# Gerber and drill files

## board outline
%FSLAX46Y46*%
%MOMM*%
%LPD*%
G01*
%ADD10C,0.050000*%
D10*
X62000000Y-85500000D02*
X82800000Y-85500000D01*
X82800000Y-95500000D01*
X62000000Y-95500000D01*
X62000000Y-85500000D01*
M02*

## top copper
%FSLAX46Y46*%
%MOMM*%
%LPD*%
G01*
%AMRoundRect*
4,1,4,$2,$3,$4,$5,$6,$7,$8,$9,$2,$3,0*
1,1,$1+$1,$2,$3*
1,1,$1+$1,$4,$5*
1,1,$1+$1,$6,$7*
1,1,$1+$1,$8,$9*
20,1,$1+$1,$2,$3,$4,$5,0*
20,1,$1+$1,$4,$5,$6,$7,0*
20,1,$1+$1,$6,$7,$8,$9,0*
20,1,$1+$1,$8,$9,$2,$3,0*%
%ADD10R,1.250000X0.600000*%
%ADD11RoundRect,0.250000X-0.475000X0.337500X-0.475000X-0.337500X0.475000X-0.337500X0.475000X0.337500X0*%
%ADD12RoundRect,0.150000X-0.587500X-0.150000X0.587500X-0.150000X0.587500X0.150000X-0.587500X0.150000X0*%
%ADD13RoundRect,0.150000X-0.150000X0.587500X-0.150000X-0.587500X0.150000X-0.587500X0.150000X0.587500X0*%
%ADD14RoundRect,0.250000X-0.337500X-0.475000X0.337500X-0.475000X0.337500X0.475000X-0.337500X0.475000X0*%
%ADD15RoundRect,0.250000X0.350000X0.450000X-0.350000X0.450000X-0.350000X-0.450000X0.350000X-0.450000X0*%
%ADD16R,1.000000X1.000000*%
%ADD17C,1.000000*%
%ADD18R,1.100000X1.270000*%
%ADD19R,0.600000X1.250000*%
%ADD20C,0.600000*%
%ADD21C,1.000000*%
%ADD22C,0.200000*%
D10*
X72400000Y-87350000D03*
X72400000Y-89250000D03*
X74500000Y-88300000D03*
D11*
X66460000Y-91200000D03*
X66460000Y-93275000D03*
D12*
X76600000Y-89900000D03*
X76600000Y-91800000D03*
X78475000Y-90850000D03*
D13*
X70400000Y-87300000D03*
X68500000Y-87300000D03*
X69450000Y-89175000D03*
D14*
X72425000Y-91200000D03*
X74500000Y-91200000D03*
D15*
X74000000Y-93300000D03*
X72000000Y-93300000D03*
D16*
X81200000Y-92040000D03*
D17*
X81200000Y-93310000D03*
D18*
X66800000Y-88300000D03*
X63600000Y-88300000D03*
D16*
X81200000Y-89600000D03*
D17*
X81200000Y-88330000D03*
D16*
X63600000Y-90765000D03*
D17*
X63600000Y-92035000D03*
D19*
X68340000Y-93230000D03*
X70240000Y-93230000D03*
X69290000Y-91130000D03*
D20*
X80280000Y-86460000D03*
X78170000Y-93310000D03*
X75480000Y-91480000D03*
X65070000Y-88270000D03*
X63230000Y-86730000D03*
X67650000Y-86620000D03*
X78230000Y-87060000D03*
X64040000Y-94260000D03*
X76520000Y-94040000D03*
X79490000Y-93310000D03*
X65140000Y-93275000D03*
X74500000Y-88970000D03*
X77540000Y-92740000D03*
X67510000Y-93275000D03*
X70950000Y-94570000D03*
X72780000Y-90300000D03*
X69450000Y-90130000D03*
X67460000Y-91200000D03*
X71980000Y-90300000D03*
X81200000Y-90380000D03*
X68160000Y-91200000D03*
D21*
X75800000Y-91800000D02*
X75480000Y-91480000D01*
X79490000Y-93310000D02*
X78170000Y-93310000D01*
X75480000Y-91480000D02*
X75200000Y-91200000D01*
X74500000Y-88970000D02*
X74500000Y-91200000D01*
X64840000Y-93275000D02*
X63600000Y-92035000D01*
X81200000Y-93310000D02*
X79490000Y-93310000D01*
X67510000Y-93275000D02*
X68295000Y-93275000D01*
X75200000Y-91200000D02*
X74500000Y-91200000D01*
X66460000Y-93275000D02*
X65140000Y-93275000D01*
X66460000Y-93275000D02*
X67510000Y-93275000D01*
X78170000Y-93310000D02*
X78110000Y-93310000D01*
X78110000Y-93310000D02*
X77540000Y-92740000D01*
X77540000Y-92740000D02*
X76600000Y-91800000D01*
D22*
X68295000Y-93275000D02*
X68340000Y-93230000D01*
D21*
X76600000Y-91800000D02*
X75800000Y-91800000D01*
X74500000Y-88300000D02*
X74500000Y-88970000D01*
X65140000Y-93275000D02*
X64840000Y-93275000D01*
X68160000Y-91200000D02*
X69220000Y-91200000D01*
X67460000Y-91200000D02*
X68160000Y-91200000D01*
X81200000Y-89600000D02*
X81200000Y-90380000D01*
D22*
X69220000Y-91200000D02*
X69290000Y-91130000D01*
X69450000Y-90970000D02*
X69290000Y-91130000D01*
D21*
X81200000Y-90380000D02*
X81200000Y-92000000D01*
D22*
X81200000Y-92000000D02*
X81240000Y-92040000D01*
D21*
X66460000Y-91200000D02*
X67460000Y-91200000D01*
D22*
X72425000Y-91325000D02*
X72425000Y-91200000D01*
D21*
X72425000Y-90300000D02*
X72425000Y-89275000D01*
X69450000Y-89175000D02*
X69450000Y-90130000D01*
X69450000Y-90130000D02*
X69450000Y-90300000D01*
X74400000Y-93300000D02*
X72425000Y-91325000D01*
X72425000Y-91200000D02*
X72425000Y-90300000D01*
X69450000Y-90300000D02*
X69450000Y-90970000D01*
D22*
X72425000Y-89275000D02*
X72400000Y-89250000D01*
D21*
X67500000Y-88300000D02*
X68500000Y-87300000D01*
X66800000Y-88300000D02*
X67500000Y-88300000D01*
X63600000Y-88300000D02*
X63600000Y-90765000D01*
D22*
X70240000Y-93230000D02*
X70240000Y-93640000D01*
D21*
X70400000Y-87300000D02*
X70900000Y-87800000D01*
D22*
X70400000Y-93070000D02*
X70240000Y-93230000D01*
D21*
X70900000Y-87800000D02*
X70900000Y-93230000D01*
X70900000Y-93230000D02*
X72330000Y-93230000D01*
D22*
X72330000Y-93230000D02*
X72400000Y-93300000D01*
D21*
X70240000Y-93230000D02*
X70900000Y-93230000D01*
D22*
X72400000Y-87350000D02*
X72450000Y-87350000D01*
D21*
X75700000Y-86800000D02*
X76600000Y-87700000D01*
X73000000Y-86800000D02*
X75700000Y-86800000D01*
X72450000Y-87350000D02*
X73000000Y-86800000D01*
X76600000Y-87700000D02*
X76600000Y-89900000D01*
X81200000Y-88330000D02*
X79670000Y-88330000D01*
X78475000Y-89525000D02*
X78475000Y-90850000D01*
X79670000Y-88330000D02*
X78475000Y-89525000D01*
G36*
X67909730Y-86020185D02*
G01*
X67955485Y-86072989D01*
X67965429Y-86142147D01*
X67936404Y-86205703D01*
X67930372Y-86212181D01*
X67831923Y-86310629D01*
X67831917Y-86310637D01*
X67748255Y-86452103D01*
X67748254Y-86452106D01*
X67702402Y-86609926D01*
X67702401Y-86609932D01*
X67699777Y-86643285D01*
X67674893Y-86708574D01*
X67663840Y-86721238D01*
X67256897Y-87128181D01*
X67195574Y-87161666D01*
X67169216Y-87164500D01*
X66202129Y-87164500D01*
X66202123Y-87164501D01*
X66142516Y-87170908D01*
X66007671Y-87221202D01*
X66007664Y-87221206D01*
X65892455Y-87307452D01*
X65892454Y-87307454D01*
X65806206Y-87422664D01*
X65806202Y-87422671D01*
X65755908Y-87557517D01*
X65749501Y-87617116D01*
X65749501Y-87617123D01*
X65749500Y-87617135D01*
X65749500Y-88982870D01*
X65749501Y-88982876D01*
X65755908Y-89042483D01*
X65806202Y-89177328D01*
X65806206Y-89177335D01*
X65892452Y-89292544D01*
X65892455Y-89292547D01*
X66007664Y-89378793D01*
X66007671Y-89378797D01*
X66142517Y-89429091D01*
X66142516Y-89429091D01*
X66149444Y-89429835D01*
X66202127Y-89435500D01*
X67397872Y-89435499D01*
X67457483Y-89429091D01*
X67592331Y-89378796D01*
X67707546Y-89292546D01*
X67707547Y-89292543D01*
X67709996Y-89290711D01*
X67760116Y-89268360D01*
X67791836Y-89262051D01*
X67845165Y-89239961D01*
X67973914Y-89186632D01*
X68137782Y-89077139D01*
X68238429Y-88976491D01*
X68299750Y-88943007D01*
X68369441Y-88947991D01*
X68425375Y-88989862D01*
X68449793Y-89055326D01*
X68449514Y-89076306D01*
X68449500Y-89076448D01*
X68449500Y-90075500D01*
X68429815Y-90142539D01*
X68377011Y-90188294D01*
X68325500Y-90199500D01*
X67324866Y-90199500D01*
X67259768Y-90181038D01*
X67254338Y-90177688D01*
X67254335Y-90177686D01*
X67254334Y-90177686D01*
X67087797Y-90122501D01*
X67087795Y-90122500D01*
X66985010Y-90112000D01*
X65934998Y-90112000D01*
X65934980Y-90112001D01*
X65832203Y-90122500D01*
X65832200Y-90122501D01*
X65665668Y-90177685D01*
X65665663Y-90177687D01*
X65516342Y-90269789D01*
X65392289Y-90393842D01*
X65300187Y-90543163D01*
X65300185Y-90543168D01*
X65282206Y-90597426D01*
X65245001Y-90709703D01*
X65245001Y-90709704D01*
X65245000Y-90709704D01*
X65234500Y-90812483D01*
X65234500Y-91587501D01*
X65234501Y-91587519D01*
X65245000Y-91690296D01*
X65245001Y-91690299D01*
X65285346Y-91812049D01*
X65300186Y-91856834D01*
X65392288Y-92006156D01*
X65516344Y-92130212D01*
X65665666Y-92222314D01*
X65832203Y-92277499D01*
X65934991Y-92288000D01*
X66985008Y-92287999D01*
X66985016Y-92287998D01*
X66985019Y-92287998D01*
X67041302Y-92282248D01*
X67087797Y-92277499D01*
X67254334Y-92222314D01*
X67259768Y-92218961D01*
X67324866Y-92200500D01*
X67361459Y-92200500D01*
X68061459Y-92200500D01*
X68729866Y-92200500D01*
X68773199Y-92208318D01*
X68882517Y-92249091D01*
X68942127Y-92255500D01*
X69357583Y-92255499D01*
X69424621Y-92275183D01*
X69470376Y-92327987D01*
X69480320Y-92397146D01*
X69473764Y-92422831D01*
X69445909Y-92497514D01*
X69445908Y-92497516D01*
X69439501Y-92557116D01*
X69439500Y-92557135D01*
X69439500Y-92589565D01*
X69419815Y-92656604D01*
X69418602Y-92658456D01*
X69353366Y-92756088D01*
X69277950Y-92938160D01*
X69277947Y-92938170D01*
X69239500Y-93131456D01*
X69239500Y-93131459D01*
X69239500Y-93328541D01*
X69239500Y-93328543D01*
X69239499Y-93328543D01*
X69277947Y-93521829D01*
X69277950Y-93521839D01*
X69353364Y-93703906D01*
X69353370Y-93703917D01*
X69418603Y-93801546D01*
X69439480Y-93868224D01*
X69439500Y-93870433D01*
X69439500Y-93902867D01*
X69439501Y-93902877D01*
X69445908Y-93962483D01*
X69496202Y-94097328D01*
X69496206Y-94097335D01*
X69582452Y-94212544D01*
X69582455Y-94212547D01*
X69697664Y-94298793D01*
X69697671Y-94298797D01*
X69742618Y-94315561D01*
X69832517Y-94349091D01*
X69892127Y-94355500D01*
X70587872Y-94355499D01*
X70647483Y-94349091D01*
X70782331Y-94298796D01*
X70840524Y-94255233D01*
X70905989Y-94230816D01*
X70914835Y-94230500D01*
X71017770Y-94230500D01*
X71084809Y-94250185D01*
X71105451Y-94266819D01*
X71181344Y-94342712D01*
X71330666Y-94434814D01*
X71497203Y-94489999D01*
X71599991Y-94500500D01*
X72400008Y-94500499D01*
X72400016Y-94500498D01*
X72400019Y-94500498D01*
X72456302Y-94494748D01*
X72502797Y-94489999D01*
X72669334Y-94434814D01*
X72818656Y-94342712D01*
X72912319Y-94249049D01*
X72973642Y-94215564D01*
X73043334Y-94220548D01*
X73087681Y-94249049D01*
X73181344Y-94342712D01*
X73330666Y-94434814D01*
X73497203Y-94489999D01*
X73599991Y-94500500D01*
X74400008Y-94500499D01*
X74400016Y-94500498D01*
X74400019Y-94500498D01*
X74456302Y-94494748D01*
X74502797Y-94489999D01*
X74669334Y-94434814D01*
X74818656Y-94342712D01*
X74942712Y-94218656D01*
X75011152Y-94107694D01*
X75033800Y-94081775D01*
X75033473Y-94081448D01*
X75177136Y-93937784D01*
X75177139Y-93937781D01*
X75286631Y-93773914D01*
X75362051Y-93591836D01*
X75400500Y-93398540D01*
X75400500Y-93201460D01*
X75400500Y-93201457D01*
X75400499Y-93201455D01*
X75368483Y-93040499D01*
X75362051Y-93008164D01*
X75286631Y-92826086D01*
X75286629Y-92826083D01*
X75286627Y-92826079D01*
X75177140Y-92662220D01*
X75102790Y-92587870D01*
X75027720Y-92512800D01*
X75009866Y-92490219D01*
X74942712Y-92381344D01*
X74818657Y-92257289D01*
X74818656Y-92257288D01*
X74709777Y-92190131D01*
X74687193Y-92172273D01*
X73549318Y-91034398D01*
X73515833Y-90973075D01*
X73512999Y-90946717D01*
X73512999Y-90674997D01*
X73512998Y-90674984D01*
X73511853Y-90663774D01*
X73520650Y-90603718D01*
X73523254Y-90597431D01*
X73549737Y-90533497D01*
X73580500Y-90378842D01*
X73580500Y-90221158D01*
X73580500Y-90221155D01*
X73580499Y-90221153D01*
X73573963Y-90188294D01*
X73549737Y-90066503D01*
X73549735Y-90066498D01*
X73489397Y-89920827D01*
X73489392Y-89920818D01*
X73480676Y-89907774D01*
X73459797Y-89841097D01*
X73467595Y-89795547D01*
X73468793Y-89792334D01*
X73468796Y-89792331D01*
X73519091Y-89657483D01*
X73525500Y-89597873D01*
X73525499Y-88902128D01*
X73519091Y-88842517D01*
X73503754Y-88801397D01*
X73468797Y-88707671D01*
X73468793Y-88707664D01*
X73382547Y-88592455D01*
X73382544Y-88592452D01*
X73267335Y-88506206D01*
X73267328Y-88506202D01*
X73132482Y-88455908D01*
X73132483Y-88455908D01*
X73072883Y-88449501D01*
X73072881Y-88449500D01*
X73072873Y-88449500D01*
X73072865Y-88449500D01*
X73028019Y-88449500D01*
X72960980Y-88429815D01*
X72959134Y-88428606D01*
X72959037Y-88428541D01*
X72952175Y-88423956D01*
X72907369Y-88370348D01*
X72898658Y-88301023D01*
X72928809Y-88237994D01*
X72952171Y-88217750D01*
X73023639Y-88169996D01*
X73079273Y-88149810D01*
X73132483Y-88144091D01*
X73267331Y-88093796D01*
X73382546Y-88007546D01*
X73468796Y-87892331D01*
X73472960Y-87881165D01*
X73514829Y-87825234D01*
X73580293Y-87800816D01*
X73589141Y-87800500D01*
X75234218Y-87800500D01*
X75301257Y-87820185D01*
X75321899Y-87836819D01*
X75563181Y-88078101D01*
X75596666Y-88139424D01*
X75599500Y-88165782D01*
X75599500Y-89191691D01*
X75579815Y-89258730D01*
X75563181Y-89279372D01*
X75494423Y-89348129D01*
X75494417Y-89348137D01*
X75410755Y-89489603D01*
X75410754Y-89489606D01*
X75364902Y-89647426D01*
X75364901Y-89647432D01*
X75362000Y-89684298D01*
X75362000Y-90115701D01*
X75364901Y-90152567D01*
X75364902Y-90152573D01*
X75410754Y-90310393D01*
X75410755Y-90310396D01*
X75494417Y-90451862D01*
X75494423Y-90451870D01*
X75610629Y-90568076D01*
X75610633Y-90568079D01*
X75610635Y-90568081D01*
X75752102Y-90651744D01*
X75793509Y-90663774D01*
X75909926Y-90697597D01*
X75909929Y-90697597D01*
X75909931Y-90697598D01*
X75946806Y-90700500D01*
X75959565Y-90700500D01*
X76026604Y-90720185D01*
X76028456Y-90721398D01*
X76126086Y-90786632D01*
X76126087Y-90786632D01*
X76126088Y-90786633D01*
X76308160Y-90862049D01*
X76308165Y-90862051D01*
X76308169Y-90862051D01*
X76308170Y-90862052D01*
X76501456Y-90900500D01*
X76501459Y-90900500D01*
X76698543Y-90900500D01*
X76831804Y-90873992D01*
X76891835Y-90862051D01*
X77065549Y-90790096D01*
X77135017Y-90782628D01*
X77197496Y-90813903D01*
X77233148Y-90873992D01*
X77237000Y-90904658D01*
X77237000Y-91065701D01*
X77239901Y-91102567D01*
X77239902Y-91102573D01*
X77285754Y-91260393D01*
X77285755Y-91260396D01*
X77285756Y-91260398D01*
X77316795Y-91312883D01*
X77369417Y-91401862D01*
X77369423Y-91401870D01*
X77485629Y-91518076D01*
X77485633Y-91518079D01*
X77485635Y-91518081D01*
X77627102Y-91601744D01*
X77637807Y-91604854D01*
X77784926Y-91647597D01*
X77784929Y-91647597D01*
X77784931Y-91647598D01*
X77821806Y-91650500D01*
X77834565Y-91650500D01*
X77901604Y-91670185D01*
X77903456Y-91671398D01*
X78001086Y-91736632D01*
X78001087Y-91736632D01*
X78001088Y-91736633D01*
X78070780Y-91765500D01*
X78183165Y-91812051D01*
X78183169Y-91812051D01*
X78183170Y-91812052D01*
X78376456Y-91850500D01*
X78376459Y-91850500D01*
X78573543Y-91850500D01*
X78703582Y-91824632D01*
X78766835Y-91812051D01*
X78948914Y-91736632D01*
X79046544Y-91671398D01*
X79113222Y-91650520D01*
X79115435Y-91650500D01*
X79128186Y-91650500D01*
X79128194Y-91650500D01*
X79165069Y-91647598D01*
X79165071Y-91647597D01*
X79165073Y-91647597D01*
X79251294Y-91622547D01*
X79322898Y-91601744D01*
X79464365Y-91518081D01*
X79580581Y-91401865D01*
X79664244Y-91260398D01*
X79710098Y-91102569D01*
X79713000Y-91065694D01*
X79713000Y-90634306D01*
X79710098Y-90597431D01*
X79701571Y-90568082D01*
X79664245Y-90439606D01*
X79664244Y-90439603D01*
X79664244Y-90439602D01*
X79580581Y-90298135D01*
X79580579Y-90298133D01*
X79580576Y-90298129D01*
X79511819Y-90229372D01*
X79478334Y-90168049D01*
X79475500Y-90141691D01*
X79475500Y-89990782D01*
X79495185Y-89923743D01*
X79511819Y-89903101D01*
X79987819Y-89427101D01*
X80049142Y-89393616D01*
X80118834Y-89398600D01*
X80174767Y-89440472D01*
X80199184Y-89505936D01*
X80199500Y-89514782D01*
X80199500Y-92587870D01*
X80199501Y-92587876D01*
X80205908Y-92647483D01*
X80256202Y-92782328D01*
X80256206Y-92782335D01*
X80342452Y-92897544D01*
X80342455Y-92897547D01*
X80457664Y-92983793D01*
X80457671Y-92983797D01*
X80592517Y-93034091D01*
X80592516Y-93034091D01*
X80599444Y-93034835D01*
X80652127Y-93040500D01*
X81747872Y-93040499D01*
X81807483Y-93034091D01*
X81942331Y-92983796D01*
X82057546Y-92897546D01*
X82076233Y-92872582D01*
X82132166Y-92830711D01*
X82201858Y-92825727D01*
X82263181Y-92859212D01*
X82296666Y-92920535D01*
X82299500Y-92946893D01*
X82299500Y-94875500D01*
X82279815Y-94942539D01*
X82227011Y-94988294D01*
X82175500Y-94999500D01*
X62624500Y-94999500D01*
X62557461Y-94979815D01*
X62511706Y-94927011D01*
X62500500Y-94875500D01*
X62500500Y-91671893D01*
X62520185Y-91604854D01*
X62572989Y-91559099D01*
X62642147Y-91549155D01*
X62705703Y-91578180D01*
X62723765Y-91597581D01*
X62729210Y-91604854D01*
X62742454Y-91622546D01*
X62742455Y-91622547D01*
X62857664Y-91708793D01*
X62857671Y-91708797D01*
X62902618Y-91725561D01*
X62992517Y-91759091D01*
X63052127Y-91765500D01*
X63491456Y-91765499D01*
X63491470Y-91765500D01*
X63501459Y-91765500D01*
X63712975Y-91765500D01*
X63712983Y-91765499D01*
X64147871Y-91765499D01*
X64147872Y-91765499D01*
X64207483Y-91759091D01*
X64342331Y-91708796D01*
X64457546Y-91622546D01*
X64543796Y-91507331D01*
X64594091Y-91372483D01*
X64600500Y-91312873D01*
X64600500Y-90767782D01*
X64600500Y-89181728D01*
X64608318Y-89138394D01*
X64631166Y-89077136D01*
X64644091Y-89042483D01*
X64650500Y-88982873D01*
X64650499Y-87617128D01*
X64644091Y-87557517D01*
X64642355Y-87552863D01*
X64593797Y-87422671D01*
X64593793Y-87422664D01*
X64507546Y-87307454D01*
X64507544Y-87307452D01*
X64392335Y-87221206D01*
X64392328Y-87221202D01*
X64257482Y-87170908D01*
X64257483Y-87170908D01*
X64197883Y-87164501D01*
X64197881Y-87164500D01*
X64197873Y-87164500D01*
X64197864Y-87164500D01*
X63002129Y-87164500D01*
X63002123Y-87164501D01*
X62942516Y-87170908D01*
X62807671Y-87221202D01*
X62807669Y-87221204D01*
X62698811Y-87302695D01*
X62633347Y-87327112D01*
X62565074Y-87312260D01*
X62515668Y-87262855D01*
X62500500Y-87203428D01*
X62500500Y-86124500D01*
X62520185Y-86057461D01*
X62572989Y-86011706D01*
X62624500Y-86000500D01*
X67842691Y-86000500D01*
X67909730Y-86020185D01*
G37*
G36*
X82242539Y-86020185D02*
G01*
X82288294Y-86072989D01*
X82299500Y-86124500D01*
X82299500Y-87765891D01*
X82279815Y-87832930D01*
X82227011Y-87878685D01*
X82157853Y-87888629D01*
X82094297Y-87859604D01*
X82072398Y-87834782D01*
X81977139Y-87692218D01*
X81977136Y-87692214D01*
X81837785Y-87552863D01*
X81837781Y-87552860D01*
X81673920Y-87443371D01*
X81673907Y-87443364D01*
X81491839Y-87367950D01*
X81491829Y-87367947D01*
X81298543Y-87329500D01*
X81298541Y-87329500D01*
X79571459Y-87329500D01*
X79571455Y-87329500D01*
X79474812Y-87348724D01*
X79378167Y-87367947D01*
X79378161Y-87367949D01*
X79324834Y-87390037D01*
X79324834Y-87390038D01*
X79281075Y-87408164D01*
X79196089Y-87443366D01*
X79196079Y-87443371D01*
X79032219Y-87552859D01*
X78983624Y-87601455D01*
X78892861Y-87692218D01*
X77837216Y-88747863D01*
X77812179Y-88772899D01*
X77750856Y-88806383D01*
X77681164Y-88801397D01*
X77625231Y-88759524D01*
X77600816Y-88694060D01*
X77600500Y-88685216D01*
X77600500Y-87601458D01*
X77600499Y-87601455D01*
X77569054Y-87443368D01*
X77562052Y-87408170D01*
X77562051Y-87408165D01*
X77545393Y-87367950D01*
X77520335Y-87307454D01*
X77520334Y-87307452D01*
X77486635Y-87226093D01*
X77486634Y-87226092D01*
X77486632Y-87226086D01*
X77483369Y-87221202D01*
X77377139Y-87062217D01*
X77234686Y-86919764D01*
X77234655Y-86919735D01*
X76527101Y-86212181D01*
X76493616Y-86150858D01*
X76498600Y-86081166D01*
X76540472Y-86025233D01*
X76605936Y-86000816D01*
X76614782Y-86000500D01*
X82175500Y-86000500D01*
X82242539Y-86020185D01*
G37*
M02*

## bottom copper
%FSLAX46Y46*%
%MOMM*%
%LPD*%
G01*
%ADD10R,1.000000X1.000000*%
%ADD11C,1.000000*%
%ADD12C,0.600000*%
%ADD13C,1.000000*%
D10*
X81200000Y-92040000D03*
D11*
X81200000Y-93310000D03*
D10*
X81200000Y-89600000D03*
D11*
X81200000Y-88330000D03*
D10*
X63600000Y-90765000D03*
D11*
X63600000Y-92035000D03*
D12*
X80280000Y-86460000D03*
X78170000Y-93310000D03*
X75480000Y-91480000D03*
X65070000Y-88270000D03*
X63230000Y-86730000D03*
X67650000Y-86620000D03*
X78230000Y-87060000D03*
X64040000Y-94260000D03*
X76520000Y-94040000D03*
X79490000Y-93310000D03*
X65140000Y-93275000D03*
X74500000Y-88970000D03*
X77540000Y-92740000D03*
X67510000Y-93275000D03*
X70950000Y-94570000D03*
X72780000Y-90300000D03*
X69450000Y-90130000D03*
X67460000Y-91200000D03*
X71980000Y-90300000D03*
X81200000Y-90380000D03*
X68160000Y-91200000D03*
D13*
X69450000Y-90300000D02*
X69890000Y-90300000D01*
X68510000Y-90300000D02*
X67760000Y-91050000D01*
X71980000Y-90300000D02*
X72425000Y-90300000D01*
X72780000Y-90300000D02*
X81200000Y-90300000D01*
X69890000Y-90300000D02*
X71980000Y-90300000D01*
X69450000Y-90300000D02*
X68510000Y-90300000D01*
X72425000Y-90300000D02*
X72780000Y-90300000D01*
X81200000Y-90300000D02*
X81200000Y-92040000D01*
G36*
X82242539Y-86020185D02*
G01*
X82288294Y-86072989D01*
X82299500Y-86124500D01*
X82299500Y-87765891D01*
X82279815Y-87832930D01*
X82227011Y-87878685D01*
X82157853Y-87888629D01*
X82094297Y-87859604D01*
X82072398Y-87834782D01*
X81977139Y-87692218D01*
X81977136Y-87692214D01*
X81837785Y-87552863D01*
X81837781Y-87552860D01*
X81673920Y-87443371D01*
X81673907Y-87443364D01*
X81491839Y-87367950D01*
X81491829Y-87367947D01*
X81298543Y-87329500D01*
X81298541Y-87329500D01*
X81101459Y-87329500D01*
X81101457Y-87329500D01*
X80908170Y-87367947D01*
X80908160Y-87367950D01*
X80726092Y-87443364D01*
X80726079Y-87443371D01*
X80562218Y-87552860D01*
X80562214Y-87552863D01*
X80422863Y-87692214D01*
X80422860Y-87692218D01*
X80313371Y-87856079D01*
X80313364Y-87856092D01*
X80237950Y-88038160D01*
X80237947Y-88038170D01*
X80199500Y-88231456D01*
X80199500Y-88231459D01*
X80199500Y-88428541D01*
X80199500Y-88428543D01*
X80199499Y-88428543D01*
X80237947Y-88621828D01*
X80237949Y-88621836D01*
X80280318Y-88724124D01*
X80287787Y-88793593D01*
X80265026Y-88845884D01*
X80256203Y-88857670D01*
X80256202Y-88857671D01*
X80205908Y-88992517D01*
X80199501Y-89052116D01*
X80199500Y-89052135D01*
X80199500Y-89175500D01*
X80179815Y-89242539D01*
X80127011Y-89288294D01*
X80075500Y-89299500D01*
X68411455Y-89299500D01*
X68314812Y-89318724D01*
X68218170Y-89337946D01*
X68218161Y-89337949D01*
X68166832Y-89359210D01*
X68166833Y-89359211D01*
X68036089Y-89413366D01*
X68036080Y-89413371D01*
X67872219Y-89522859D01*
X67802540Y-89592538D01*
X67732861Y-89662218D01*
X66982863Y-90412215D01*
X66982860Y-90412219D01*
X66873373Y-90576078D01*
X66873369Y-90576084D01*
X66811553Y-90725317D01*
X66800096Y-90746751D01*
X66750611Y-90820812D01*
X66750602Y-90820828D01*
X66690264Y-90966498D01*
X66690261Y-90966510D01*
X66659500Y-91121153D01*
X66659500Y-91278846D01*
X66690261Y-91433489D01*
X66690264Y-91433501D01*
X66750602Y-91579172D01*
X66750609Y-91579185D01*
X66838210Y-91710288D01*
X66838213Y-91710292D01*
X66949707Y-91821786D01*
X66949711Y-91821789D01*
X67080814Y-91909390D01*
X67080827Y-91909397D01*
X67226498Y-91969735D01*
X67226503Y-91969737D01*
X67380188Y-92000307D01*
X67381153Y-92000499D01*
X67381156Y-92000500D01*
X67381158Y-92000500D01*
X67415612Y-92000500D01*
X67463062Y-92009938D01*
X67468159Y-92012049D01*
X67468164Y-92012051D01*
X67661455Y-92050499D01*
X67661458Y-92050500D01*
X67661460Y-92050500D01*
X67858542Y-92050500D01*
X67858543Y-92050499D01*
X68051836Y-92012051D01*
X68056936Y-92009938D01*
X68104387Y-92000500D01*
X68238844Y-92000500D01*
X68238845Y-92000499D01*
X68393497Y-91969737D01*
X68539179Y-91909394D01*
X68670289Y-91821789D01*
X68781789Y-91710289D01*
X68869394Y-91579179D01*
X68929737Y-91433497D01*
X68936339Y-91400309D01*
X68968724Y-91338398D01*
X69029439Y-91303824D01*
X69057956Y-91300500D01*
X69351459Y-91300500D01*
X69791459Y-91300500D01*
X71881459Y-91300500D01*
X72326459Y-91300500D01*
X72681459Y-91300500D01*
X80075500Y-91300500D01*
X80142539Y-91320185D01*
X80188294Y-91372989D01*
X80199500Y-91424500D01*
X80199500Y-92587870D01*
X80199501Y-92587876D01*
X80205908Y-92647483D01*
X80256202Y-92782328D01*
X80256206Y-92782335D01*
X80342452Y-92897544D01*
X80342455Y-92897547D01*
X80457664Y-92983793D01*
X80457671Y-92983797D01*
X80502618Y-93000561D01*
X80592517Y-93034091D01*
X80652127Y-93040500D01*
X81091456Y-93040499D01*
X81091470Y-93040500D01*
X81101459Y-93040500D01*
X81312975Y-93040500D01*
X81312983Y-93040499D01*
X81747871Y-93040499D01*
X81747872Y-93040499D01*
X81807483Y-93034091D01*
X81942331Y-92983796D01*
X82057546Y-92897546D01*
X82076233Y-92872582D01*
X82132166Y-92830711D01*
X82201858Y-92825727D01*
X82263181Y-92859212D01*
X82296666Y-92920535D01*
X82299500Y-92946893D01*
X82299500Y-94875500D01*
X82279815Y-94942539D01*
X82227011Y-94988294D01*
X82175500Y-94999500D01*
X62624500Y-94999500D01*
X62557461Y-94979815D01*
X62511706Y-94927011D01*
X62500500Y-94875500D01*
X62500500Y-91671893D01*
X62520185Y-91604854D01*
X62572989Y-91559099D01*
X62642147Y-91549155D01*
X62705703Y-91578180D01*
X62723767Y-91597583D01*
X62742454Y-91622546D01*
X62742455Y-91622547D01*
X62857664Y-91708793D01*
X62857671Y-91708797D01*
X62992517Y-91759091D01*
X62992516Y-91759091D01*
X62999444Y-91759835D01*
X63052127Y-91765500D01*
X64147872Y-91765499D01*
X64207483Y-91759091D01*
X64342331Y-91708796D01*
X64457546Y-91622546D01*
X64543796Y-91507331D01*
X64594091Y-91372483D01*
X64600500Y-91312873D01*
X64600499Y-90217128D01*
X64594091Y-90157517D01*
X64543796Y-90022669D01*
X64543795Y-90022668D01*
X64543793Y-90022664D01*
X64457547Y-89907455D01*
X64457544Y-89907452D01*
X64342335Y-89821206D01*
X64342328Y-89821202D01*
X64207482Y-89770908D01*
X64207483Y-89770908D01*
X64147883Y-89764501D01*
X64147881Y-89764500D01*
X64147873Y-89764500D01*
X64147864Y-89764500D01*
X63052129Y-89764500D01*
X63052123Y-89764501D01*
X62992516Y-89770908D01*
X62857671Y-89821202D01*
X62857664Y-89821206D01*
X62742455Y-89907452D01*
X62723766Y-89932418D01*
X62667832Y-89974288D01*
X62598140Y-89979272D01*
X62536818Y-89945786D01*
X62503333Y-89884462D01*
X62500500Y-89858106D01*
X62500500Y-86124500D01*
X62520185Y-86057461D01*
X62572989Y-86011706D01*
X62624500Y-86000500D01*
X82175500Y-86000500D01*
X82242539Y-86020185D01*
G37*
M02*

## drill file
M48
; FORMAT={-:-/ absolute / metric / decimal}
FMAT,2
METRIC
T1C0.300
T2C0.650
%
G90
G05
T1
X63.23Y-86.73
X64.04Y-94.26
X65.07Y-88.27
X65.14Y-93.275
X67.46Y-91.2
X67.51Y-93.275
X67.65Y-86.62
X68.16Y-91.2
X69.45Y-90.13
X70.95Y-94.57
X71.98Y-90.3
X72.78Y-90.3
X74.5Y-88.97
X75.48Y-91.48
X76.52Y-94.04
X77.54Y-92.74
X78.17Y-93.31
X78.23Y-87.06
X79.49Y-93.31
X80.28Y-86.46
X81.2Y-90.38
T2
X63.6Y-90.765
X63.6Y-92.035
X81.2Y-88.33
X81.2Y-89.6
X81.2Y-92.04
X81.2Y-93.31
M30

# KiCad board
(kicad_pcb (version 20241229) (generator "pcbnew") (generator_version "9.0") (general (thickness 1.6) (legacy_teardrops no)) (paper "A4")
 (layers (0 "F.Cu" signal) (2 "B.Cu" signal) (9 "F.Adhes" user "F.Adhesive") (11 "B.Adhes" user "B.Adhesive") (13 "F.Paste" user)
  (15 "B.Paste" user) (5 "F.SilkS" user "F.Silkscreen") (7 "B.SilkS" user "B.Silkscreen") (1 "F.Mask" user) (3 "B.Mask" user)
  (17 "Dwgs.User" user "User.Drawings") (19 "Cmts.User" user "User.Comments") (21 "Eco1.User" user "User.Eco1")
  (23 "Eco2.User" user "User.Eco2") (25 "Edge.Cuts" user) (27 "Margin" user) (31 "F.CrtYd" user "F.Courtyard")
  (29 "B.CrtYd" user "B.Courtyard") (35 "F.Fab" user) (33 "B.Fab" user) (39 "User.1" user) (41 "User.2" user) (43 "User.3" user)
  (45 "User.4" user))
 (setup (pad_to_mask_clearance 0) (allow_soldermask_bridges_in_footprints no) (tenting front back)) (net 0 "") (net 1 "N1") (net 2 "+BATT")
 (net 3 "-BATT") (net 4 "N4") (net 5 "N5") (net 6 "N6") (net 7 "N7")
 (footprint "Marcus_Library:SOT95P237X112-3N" (layer "F.Cu") (at 73.45 88.3)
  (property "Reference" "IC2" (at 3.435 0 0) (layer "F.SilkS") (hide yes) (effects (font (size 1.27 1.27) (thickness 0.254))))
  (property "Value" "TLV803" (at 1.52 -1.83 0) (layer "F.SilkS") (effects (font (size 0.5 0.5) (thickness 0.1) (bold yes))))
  (pad "1" smd rect (at -1.05 -0.95 90) (size 0.6 1.25) (layers "F.Cu" "F.Mask" "F.Paste") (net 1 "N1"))
  (pad "2" smd rect (at -1.05 0.95 90) (size 0.6 1.25) (layers "F.Cu" "F.Mask" "F.Paste") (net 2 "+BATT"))
  (pad "3" smd rect (at 1.05 0 90) (size 0.6 1.25) (layers "F.Cu" "F.Mask" "F.Paste") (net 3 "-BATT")))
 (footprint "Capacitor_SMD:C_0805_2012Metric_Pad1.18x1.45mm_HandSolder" (layer "F.Cu") (at 66.46 92.2375 -90)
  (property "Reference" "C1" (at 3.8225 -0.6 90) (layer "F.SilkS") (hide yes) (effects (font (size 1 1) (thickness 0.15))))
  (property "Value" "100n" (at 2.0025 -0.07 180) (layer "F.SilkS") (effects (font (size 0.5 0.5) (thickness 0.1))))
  (pad "1" smd roundrect (at -1.0375 0 270) (size 1.175 1.45) (layers "F.Cu" "F.Mask" "F.Paste") (roundrect_rratio 0.212766) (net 2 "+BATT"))
  (pad "2" smd roundrect (at 1.0375 0 270) (size 1.175 1.45) (layers "F.Cu" "F.Mask" "F.Paste") (roundrect_rratio 0.212766) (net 3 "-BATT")))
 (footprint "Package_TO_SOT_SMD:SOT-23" (layer "F.Cu") (at 77.5375 90.85)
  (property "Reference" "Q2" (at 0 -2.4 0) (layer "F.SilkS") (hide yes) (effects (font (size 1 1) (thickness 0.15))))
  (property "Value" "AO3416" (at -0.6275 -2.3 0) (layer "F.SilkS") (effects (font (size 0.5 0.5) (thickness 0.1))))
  (pad "1" smd roundrect (at -0.9375 -0.95) (size 1.475 0.6) (layers "F.Cu" "F.Mask" "F.Paste") (roundrect_rratio 0.25) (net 1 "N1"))
  (pad "2" smd roundrect (at -0.9375 0.95) (size 1.475 0.6) (layers "F.Cu" "F.Mask" "F.Paste") (roundrect_rratio 0.25) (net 3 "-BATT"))
  (pad "3" smd roundrect (at 0.9375 0) (size 1.475 0.6) (layers "F.Cu" "F.Mask" "F.Paste") (roundrect_rratio 0.25) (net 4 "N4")))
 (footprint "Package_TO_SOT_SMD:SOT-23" (layer "F.Cu") (at 69.45 88.2375 -90)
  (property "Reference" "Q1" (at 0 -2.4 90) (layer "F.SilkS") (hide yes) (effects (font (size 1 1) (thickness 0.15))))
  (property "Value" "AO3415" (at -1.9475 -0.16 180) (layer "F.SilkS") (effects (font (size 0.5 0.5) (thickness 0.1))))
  (pad "1" smd roundrect (at -0.9375 -0.95 270) (size 1.475 0.6) (layers "F.Cu" "F.Mask" "F.Paste") (roundrect_rratio 0.25) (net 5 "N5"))
  (pad "2" smd roundrect (at -0.9375 0.95 270) (size 1.475 0.6) (layers "F.Cu" "F.Mask" "F.Paste") (roundrect_rratio 0.25) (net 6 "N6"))
  (pad "3" smd roundrect (at 0.9375 0 270) (size 1.475 0.6) (layers "F.Cu" "F.Mask" "F.Paste") (roundrect_rratio 0.25) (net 2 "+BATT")))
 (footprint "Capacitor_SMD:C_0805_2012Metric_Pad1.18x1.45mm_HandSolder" (layer "F.Cu") (at 73.4625 91.2)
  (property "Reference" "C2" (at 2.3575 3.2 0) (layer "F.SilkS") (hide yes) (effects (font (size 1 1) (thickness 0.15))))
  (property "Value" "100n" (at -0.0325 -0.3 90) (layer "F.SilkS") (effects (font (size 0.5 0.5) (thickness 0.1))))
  (pad "1" smd roundrect (at -1.0375 0) (size 1.175 1.45) (layers "F.Cu" "F.Mask" "F.Paste") (roundrect_rratio 0.212766) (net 2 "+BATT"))
  (pad "2" smd roundrect (at 1.0375 0) (size 1.175 1.45) (layers "F.Cu" "F.Mask" "F.Paste") (roundrect_rratio 0.212766) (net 3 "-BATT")))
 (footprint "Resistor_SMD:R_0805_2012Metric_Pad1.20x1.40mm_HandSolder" (layer "F.Cu") (at 73 93.3 180)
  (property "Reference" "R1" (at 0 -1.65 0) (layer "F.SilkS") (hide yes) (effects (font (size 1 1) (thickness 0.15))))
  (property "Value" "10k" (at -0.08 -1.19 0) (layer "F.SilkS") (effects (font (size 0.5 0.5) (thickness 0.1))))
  (pad "1" smd roundrect (at -1 0 180) (size 1.2 1.4) (layers "F.Cu" "F.Mask" "F.Paste") (roundrect_rratio 0.208333) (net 2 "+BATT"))
  (pad "2" smd roundrect (at 1 0 180) (size 1.2 1.4) (layers "F.Cu" "F.Mask" "F.Paste") (roundrect_rratio 0.208333) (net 5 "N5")))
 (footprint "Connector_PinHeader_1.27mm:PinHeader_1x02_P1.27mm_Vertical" (layer "F.Cu") (at 81.2 92.04)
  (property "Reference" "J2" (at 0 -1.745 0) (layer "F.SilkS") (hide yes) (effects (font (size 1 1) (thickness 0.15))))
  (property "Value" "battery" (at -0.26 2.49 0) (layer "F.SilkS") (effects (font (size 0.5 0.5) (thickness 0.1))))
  (pad "1" thru_hole rect (at 0 0) (size 1 1) (drill 0.65) (layers "*.Cu" "*.Mask") (remove_unused_layers no) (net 2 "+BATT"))
  (pad "2" thru_hole circle (at 0 1.27) (size 1 1) (drill 0.65) (layers "*.Cu" "*.Mask") (remove_unused_layers no) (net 3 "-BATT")))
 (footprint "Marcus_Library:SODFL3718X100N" (layer "F.Cu") (at 65.2 88.3 180)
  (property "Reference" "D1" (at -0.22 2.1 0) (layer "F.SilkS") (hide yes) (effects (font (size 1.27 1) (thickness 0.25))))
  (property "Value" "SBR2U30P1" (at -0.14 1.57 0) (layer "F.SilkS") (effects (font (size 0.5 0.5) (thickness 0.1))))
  (pad "1" smd rect (at -1.6 0 180) (size 1.1 1.27) (layers "F.Cu" "F.Mask" "F.Paste") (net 6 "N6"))
  (pad "2" smd rect (at 1.6 0 180) (size 1.1 1.27) (layers "F.Cu" "F.Mask" "F.Paste") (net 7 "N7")))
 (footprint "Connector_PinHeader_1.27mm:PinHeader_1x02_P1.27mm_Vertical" (layer "F.Cu") (at 81.2 89.6 180)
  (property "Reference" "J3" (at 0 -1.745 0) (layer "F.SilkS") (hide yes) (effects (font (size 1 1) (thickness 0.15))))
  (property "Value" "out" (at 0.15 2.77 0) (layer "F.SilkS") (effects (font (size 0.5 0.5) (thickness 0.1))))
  (pad "1" thru_hole rect (at 0 0 180) (size 1 1) (drill 0.65) (layers "*.Cu" "*.Mask") (remove_unused_layers no) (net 2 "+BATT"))
  (pad "2" thru_hole circle (at 0 1.27 180) (size 1 1) (drill 0.65) (layers "*.Cu" "*.Mask") (remove_unused_layers no) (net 4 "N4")))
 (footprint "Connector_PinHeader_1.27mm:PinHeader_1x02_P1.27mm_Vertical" (layer "F.Cu") (at 63.6 90.765)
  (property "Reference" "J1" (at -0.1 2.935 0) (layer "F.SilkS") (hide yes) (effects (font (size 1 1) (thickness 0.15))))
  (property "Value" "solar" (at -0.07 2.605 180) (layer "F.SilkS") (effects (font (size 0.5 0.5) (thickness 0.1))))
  (pad "1" thru_hole rect (at 0 0) (size 1 1) (drill 0.65) (layers "*.Cu" "*.Mask") (remove_unused_layers no) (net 7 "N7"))
  (pad "2" thru_hole circle (at 0 1.27) (size 1 1) (drill 0.65) (layers "*.Cu" "*.Mask") (remove_unused_layers no) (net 3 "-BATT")))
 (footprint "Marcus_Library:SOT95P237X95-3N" (layer "F.Cu") (at 69.29 92.18 90)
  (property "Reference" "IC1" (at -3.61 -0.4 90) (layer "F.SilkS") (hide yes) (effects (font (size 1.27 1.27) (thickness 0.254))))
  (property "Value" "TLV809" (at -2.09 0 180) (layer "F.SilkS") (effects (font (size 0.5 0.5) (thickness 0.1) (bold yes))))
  (pad "1" smd rect (at -1.05 -0.95 180) (size 0.6 1.25) (layers "F.Cu" "F.Mask" "F.Paste") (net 3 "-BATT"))
  (pad "2" smd rect (at -1.05 0.95 180) (size 0.6 1.25) (layers "F.Cu" "F.Mask" "F.Paste") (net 5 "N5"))
  (pad "3" smd rect (at 1.05 0 180) (size 0.6 1.25) (layers "F.Cu" "F.Mask" "F.Paste") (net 2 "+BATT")))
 (gr_rect (start 62 85.5) (end 82.8 95.5) (stroke (width 0.05) (type default)) (fill no) (layer "Edge.Cuts"))
 (segment (start 75.8 91.8) (end 75.48 91.48) (width 1) (layer "F.Cu") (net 3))
 (segment (start 79.49 93.31) (end 78.17 93.31) (width 1) (layer "F.Cu") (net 3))
 (segment (start 75.48 91.48) (end 75.2 91.2) (width 1) (layer "F.Cu") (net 3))
 (segment (start 74.5 88.97) (end 74.5 91.2) (width 1) (layer "F.Cu") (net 3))
 (segment (start 64.84 93.275) (end 63.6 92.035) (width 1) (layer "F.Cu") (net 3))
 (segment (start 81.2 93.31) (end 79.49 93.31) (width 1) (layer "F.Cu") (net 3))
 (segment (start 67.51 93.275) (end 68.295 93.275) (width 1) (layer "F.Cu") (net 3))
 (segment (start 75.2 91.2) (end 74.5 91.2) (width 1) (layer "F.Cu") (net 3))
 (segment (start 66.46 93.275) (end 65.14 93.275) (width 1) (layer "F.Cu") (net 3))
 (segment (start 66.46 93.275) (end 67.51 93.275) (width 1) (layer "F.Cu") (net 3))
 (segment (start 78.17 93.31) (end 78.11 93.31) (width 1) (layer "F.Cu") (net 3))
 (segment (start 78.11 93.31) (end 77.54 92.74) (width 1) (layer "F.Cu") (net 3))
 (segment (start 77.54 92.74) (end 76.6 91.8) (width 1) (layer "F.Cu") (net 3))
 (segment (start 68.295 93.275) (end 68.34 93.23) (width 0.2) (layer "F.Cu") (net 3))
 (segment (start 76.6 91.8) (end 75.8 91.8) (width 1) (layer "F.Cu") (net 3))
 (segment (start 74.5 88.3) (end 74.5 88.97) (width 1) (layer "F.Cu") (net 3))
 (segment (start 65.14 93.275) (end 64.84 93.275) (width 1) (layer "F.Cu") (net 3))
 (via (at 80.28 86.46) (size 0.6) (drill 0.3) (layers "F.Cu" "B.Cu") (free yes) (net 3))
 (via (at 78.17 93.31) (size 0.6) (drill 0.3) (layers "F.Cu" "B.Cu") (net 3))
 (via (at 75.48 91.48) (size 0.6) (drill 0.3) (layers "F.Cu" "B.Cu") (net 3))
 (via (at 65.07 88.27) (size 0.6) (drill 0.3) (layers "F.Cu" "B.Cu") (free yes) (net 3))
 (via (at 63.23 86.73) (size 0.6) (drill 0.3) (layers "F.Cu" "B.Cu") (free yes) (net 3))
 (via (at 67.65 86.62) (size 0.6) (drill 0.3) (layers "F.Cu" "B.Cu") (free yes) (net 3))
 (via (at 78.23 87.06) (size 0.6) (drill 0.3) (layers "F.Cu" "B.Cu") (free yes) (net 3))
 (via (at 64.04 94.26) (size 0.6) (drill 0.3) (layers "F.Cu" "B.Cu") (free yes) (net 3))
 (via (at 76.52 94.04) (size 0.6) (drill 0.3) (layers "F.Cu" "B.Cu") (free yes) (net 3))
 (via (at 79.49 93.31) (size 0.6) (drill 0.3) (layers "F.Cu" "B.Cu") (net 3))
 (via (at 65.14 93.275) (size 0.6) (drill 0.3) (layers "F.Cu" "B.Cu") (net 3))
 (via (at 74.5 88.97) (size 0.6) (drill 0.3) (layers "F.Cu" "B.Cu") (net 3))
 (via (at 77.54 92.74) (size 0.6) (drill 0.3) (layers "F.Cu" "B.Cu") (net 3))
 (via (at 67.51 93.275) (size 0.6) (drill 0.3) (layers "F.Cu" "B.Cu") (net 3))
 (via (at 70.95 94.57) (size 0.6) (drill 0.3) (layers "F.Cu" "B.Cu") (free yes) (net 3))
 (segment (start 68.16 91.2) (end 69.22 91.2) (width 1) (layer "F.Cu") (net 2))
 (segment (start 67.46 91.2) (end 68.16 91.2) (width 1) (layer "F.Cu") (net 2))
 (segment (start 81.2 89.6) (end 81.2 90.38) (width 1) (layer "F.Cu") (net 2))
 (segment (start 69.22 91.2) (end 69.29 91.13) (width 0.2) (layer "F.Cu") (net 2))
 (segment (start 69.45 90.97) (end 69.29 91.13) (width 0.2) (layer "F.Cu") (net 2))
 (segment (start 81.2 90.38) (end 81.2 92) (width 1) (layer "F.Cu") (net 2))
 (segment (start 81.2 92) (end 81.24 92.04) (width 0.2) (layer "F.Cu") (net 2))
 (segment (start 66.46 91.2) (end 67.46 91.2) (width 1) (layer "F.Cu") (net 2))
 (segment (start 72.425 91.325) (end 72.425 91.2) (width 0.2) (layer "F.Cu") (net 2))
 (segment (start 72.425 90.3) (end 72.425 89.275) (width 1) (layer "F.Cu") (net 2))
 (segment (start 69.45 89.175) (end 69.45 90.13) (width 1) (layer "F.Cu") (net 2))
 (segment (start 69.45 90.13) (end 69.45 90.3) (width 1) (layer "F.Cu") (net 2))
 (segment (start 74.4 93.3) (end 72.425 91.325) (width 1) (layer "F.Cu") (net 2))
 (segment (start 72.425 91.2) (end 72.425 90.3) (width 1) (layer "F.Cu") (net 2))
 (segment (start 69.45 90.3) (end 69.45 90.97) (width 1) (layer "F.Cu") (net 2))
 (segment (start 72.425 89.275) (end 72.4 89.25) (width 0.2) (layer "F.Cu") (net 2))
 (via (at 72.78 90.3) (size 0.6) (drill 0.3) (layers "F.Cu" "B.Cu") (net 2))
 (via (at 69.45 90.13) (size 0.6) (drill 0.3) (layers "F.Cu" "B.Cu") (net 2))
 (via (at 67.46 91.2) (size 0.6) (drill 0.3) (layers "F.Cu" "B.Cu") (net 2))
 (via (at 71.98 90.3) (size 0.6) (drill 0.3) (layers "F.Cu" "B.Cu") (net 2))
 (via (at 81.2 90.38) (size 0.6) (drill 0.3) (layers "F.Cu" "B.Cu") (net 2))
 (via (at 68.16 91.2) (size 0.6) (drill 0.3) (layers "F.Cu" "B.Cu") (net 2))
 (segment (start 69.45 90.3) (end 69.89 90.3) (width 1) (layer "B.Cu") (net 2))
 (segment (start 68.51 90.3) (end 67.76 91.05) (width 1) (layer "B.Cu") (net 2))
 (segment (start 71.98 90.3) (end 72.425 90.3) (width 1) (layer "B.Cu") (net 2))
 (segment (start 72.78 90.3) (end 81.2 90.3) (width 1) (layer "B.Cu") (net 2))
 (segment (start 69.89 90.3) (end 71.98 90.3) (width 1) (layer "B.Cu") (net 2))
 (segment (start 69.45 90.3) (end 68.51 90.3) (width 1) (layer "B.Cu") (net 2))
 (segment (start 72.425 90.3) (end 72.78 90.3) (width 1) (layer "B.Cu") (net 2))
 (segment (start 81.2 90.3) (end 81.2 92.04) (width 1) (layer "B.Cu") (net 2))
 (segment (start 67.5 88.3) (end 68.5 87.3) (width 1) (layer "F.Cu") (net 6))
 (segment (start 66.8 88.3) (end 67.5 88.3) (width 1) (layer "F.Cu") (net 6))
 (segment (start 63.6 88.3) (end 63.6 90.765) (width 1) (layer "F.Cu") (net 7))
 (segment (start 70.24 93.23) (end 70.24 93.64) (width 0.2) (layer "F.Cu") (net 5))
 (segment (start 70.4 87.3) (end 70.9 87.8) (width 1) (layer "F.Cu") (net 5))
 (segment (start 70.4 93.07) (end 70.24 93.23) (width 0.2) (layer "F.Cu") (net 5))
 (segment (start 70.9 87.8) (end 70.9 93.23) (width 1) (layer "F.Cu") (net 5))
 (segment (start 70.9 93.23) (end 72.33 93.23) (width 1) (layer "F.Cu") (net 5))
 (segment (start 72.33 93.23) (end 72.4 93.3) (width 0.2) (layer "F.Cu") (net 5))
 (segment (start 70.24 93.23) (end 70.9 93.23) (width 1) (layer "F.Cu") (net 5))
 (segment (start 72.4 87.35) (end 72.45 87.35) (width 0.2) (layer "F.Cu") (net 1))
 (segment (start 75.7 86.8) (end 76.6 87.7) (width 1) (layer "F.Cu") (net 1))
 (segment (start 73 86.8) (end 75.7 86.8) (width 1) (layer "F.Cu") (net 1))
 (segment (start 72.45 87.35) (end 73 86.8) (width 1) (layer "F.Cu") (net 1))
 (segment (start 76.6 87.7) (end 76.6 89.9) (width 1) (layer "F.Cu") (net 1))
 (segment (start 81.2 88.33) (end 79.67 88.33) (width 1) (layer "F.Cu") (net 4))
 (segment (start 78.475 89.525) (end 78.475 90.85) (width 1) (layer "F.Cu") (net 4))
 (segment (start 79.67 88.33) (end 78.475 89.525) (width 1) (layer "F.Cu") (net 4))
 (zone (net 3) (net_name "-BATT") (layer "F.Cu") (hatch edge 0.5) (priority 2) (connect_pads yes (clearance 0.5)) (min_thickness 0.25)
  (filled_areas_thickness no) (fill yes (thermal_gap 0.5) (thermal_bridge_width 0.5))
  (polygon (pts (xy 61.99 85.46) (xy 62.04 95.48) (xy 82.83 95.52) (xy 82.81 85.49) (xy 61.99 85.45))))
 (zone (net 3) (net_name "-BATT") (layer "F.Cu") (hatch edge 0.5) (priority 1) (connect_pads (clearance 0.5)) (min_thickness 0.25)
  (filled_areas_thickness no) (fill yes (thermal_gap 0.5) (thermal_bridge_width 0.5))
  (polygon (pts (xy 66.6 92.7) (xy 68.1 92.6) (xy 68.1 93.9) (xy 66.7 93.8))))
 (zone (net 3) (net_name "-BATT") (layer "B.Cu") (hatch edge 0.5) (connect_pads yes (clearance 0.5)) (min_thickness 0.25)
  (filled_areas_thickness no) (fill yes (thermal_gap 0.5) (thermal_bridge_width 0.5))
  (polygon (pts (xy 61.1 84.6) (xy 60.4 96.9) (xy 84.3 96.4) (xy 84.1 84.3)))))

